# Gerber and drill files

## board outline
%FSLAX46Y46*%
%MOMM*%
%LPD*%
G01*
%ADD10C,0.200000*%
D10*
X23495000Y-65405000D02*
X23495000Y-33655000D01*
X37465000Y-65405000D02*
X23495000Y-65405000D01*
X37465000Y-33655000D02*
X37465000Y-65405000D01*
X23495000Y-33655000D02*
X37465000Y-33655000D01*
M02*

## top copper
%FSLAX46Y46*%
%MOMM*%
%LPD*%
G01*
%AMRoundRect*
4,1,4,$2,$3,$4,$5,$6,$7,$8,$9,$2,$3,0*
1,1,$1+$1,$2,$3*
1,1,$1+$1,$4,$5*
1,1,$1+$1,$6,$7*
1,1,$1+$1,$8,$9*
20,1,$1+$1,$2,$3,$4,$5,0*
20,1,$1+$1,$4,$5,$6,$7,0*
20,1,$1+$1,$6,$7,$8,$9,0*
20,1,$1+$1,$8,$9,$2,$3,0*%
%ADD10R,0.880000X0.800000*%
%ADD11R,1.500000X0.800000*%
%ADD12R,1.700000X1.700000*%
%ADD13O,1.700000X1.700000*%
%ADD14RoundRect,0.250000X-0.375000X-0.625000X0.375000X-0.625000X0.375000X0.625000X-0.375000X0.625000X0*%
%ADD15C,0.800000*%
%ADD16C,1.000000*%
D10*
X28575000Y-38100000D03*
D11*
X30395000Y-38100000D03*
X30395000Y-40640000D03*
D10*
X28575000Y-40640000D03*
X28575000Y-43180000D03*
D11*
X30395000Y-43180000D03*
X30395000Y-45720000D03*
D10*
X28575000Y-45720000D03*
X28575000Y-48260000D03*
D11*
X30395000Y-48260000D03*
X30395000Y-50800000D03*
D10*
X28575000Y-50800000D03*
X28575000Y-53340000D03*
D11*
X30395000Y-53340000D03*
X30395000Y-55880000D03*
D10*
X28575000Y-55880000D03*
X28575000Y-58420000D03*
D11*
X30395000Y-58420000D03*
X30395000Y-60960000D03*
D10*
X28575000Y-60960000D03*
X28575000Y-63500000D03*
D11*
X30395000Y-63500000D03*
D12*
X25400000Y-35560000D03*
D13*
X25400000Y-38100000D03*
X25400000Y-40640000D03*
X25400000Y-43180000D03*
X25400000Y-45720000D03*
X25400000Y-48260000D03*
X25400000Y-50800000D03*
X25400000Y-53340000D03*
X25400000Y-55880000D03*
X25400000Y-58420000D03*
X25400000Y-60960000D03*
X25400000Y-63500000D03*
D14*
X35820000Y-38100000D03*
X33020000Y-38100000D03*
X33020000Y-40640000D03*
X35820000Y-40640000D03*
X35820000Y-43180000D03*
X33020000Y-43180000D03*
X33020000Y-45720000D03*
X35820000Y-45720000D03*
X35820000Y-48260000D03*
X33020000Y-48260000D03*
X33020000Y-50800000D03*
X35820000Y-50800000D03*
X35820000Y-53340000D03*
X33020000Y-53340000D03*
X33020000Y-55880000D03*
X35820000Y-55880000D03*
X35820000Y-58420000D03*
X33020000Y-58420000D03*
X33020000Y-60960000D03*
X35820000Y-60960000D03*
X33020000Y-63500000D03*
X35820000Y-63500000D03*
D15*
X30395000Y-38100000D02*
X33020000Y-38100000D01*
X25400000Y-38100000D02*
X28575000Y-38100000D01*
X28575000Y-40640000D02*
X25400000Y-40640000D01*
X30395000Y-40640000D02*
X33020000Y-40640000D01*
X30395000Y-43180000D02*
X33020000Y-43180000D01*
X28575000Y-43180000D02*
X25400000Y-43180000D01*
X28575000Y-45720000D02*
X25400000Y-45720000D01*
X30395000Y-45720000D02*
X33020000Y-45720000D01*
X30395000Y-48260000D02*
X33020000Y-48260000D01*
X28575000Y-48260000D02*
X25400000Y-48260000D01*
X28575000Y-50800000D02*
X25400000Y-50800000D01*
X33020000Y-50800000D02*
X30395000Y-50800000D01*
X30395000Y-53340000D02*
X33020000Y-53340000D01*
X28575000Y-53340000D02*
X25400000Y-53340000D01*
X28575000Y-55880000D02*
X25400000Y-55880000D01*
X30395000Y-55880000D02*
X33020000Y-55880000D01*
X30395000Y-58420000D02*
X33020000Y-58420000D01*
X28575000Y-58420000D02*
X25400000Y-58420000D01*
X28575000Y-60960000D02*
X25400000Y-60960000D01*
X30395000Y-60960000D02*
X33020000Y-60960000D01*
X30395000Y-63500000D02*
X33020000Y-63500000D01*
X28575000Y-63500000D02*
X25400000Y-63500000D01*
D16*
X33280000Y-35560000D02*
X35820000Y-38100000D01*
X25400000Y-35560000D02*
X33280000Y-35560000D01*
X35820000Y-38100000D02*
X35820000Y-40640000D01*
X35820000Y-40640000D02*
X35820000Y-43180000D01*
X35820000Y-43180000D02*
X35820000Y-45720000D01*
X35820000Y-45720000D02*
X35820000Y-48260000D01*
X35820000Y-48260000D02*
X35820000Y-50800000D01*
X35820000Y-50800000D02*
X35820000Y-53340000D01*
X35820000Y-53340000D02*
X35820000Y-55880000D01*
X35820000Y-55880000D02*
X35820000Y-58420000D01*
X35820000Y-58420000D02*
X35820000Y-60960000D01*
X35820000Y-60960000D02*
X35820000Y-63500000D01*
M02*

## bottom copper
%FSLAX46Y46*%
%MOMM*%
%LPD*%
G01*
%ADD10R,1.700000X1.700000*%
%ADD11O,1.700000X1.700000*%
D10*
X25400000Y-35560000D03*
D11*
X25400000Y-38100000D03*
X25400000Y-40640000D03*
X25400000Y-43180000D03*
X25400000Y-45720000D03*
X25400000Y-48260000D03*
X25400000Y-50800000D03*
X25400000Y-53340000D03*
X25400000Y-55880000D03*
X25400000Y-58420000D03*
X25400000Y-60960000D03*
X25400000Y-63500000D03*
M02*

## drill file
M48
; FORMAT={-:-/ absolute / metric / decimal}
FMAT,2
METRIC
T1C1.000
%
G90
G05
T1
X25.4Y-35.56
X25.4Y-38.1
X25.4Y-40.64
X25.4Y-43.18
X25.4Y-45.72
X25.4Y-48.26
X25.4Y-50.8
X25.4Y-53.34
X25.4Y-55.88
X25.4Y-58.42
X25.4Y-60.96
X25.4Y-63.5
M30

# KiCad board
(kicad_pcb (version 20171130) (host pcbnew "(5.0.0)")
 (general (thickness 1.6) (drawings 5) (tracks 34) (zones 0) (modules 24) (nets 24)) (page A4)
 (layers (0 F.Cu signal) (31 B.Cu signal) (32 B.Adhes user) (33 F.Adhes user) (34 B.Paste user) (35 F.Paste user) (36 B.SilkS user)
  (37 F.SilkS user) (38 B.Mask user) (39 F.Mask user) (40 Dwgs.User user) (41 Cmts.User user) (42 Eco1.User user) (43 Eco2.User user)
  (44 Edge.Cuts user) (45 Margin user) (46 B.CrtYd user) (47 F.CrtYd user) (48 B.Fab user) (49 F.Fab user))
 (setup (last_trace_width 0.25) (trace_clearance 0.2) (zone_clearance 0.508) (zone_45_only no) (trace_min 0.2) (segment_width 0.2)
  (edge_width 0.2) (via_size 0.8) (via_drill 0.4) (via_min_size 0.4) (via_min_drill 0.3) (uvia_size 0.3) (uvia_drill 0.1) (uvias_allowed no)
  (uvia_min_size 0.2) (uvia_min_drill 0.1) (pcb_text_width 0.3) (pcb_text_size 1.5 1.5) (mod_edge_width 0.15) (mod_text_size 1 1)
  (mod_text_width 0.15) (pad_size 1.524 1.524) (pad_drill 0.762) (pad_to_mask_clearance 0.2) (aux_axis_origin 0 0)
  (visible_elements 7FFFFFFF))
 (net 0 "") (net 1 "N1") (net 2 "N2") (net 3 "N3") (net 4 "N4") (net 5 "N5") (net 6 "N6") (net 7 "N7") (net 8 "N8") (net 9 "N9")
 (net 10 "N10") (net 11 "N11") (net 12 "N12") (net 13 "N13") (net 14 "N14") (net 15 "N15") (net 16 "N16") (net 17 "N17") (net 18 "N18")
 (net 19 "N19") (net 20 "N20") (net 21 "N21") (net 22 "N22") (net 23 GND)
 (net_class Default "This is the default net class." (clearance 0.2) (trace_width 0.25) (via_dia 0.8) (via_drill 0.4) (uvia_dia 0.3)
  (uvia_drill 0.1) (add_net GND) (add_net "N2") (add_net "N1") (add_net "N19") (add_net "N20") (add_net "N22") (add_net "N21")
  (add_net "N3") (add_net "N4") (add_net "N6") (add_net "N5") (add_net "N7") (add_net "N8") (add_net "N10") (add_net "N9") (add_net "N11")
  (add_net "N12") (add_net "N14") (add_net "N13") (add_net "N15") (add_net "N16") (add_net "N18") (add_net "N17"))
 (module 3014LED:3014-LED (layer F.Cu) (at 28.575 38.1)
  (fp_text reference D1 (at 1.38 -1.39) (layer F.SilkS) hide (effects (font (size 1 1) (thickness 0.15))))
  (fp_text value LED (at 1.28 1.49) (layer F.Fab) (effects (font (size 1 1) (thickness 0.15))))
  (pad 2 smd rect (at 0 0) (size 0.88 0.8) (layers F.Cu F.Paste F.Mask) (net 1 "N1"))
  (pad 1 smd rect (at 1.82 0) (size 1.5 0.8) (layers F.Cu F.Paste F.Mask) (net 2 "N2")))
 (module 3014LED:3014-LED (layer F.Cu) (at 28.575 40.64)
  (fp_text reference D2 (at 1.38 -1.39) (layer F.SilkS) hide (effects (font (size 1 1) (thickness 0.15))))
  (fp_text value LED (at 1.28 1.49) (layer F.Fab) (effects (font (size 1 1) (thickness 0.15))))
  (pad 1 smd rect (at 1.82 0) (size 1.5 0.8) (layers F.Cu F.Paste F.Mask) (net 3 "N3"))
  (pad 2 smd rect (at 0 0) (size 0.88 0.8) (layers F.Cu F.Paste F.Mask) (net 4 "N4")))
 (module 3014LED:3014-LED (layer F.Cu) (at 28.575 43.18)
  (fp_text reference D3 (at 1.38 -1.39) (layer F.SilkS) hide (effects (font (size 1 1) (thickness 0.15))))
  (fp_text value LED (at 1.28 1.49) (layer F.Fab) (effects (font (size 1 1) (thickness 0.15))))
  (pad 2 smd rect (at 0 0) (size 0.88 0.8) (layers F.Cu F.Paste F.Mask) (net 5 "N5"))
  (pad 1 smd rect (at 1.82 0) (size 1.5 0.8) (layers F.Cu F.Paste F.Mask) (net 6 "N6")))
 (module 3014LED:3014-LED (layer F.Cu) (at 28.575 45.72)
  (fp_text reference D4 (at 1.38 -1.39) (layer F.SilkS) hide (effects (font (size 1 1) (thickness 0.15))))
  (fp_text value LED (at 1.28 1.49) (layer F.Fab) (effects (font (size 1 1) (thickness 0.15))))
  (pad 1 smd rect (at 1.82 0) (size 1.5 0.8) (layers F.Cu F.Paste F.Mask) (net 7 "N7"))
  (pad 2 smd rect (at 0 0) (size 0.88 0.8) (layers F.Cu F.Paste F.Mask) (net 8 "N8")))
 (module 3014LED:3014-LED (layer F.Cu) (at 28.575 48.26)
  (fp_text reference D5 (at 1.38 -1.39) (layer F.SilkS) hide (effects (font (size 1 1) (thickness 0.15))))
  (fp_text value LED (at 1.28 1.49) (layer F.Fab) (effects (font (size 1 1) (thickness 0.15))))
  (pad 2 smd rect (at 0 0) (size 0.88 0.8) (layers F.Cu F.Paste F.Mask) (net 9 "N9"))
  (pad 1 smd rect (at 1.82 0) (size 1.5 0.8) (layers F.Cu F.Paste F.Mask) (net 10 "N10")))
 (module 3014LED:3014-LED (layer F.Cu) (at 28.575 50.8)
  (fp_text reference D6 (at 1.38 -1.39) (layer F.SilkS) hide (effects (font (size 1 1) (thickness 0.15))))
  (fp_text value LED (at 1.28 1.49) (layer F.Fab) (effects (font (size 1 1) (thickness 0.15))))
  (pad 1 smd rect (at 1.82 0) (size 1.5 0.8) (layers F.Cu F.Paste F.Mask) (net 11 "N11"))
  (pad 2 smd rect (at 0 0) (size 0.88 0.8) (layers F.Cu F.Paste F.Mask) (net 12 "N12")))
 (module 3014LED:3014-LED (layer F.Cu) (at 28.575 53.34)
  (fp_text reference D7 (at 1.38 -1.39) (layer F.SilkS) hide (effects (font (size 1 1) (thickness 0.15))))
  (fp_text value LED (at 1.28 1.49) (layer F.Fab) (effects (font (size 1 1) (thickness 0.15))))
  (pad 2 smd rect (at 0 0) (size 0.88 0.8) (layers F.Cu F.Paste F.Mask) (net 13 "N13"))
  (pad 1 smd rect (at 1.82 0) (size 1.5 0.8) (layers F.Cu F.Paste F.Mask) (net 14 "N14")))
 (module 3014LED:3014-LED (layer F.Cu) (at 28.575 55.88)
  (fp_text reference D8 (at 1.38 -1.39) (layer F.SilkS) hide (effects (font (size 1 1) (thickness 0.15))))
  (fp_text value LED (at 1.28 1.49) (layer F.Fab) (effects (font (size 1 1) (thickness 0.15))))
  (pad 1 smd rect (at 1.82 0) (size 1.5 0.8) (layers F.Cu F.Paste F.Mask) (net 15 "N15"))
  (pad 2 smd rect (at 0 0) (size 0.88 0.8) (layers F.Cu F.Paste F.Mask) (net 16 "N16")))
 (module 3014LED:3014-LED (layer F.Cu) (at 28.575 58.42)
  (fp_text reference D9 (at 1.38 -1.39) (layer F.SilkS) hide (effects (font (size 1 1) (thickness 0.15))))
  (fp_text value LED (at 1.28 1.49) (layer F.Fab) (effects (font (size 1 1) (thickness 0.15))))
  (pad 2 smd rect (at 0 0) (size 0.88 0.8) (layers F.Cu F.Paste F.Mask) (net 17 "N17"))
  (pad 1 smd rect (at 1.82 0) (size 1.5 0.8) (layers F.Cu F.Paste F.Mask) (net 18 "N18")))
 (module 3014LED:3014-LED (layer F.Cu) (at 28.575 60.96)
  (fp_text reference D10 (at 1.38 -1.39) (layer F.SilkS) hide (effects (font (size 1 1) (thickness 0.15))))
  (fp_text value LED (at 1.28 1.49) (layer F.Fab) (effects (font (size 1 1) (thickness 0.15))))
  (pad 1 smd rect (at 1.82 0) (size 1.5 0.8) (layers F.Cu F.Paste F.Mask) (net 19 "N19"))
  (pad 2 smd rect (at 0 0) (size 0.88 0.8) (layers F.Cu F.Paste F.Mask) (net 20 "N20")))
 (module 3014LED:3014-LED (layer F.Cu) (at 28.575 63.5)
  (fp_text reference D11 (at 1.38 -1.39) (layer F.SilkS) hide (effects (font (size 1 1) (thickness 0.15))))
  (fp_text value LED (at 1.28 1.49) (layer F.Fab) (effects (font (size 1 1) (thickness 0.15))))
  (pad 2 smd rect (at 0 0) (size 0.88 0.8) (layers F.Cu F.Paste F.Mask) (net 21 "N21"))
  (pad 1 smd rect (at 1.82 0) (size 1.5 0.8) (layers F.Cu F.Paste F.Mask) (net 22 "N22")))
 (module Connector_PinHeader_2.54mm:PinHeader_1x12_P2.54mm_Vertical (layer F.Cu) (at 25.4 35.56)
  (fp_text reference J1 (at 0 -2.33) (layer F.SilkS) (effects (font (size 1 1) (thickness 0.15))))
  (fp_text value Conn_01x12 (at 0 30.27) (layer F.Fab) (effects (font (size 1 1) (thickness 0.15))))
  (pad 1 thru_hole rect (at 0 0) (size 1.7 1.7) (drill 1) (layers *.Cu *.Mask) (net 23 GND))
  (pad 2 thru_hole oval (at 0 2.54) (size 1.7 1.7) (drill 1) (layers *.Cu *.Mask) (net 1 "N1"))
  (pad 3 thru_hole oval (at 0 5.08) (size 1.7 1.7) (drill 1) (layers *.Cu *.Mask) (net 4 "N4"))
  (pad 4 thru_hole oval (at 0 7.62) (size 1.7 1.7) (drill 1) (layers *.Cu *.Mask) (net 5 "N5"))
  (pad 5 thru_hole oval (at 0 10.16) (size 1.7 1.7) (drill 1) (layers *.Cu *.Mask) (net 8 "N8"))
  (pad 6 thru_hole oval (at 0 12.7) (size 1.7 1.7) (drill 1) (layers *.Cu *.Mask) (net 9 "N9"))
  (pad 7 thru_hole oval (at 0 15.24) (size 1.7 1.7) (drill 1) (layers *.Cu *.Mask) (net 12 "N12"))
  (pad 8 thru_hole oval (at 0 17.78) (size 1.7 1.7) (drill 1) (layers *.Cu *.Mask) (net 13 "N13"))
  (pad 9 thru_hole oval (at 0 20.32) (size 1.7 1.7) (drill 1) (layers *.Cu *.Mask) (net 16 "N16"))
  (pad 10 thru_hole oval (at 0 22.86) (size 1.7 1.7) (drill 1) (layers *.Cu *.Mask) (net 17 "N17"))
  (pad 11 thru_hole oval (at 0 25.4) (size 1.7 1.7) (drill 1) (layers *.Cu *.Mask) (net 20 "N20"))
  (pad 12 thru_hole oval (at 0 27.94) (size 1.7 1.7) (drill 1) (layers *.Cu *.Mask) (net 21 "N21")))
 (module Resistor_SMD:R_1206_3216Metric (layer F.Cu) (at 34.42 38.1)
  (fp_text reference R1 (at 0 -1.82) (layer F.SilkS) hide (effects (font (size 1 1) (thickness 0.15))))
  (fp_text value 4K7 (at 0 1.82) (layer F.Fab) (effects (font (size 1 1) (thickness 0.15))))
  (pad 2 smd roundrect (at 1.4 0) (size 1.25 1.75) (layers F.Cu F.Paste F.Mask) (roundrect_rratio 0.2) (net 23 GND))
  (pad 1 smd roundrect (at -1.4 0) (size 1.25 1.75) (layers F.Cu F.Paste F.Mask) (roundrect_rratio 0.2) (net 2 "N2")))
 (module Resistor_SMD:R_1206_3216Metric (layer F.Cu) (at 34.42 40.64)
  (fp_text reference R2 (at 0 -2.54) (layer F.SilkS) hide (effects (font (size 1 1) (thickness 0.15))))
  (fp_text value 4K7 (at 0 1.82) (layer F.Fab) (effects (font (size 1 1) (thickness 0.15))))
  (pad 1 smd roundrect (at -1.4 0) (size 1.25 1.75) (layers F.Cu F.Paste F.Mask) (roundrect_rratio 0.2) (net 3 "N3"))
  (pad 2 smd roundrect (at 1.4 0) (size 1.25 1.75) (layers F.Cu F.Paste F.Mask) (roundrect_rratio 0.2) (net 23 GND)))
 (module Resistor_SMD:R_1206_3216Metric (layer F.Cu) (at 34.42 43.18)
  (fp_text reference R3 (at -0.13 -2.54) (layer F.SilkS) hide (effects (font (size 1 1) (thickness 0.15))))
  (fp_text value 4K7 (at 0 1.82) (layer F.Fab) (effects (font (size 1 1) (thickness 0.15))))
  (pad 2 smd roundrect (at 1.4 0) (size 1.25 1.75) (layers F.Cu F.Paste F.Mask) (roundrect_rratio 0.2) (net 23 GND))
  (pad 1 smd roundrect (at -1.4 0) (size 1.25 1.75) (layers F.Cu F.Paste F.Mask) (roundrect_rratio 0.2) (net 6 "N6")))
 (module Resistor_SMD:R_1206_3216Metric (layer F.Cu) (at 34.42 45.72)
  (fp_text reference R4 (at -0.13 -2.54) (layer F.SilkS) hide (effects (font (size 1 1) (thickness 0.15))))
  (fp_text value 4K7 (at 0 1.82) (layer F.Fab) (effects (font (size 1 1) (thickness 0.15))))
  (pad 1 smd roundrect (at -1.4 0) (size 1.25 1.75) (layers F.Cu F.Paste F.Mask) (roundrect_rratio 0.2) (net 7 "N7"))
  (pad 2 smd roundrect (at 1.4 0) (size 1.25 1.75) (layers F.Cu F.Paste F.Mask) (roundrect_rratio 0.2) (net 23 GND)))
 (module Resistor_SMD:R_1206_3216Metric (layer F.Cu) (at 34.42 48.26)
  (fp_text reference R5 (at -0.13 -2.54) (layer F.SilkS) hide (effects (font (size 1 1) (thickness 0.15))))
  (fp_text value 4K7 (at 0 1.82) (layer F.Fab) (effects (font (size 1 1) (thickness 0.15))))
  (pad 2 smd roundrect (at 1.4 0) (size 1.25 1.75) (layers F.Cu F.Paste F.Mask) (roundrect_rratio 0.2) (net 23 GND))
  (pad 1 smd roundrect (at -1.4 0) (size 1.25 1.75) (layers F.Cu F.Paste F.Mask) (roundrect_rratio 0.2) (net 10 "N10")))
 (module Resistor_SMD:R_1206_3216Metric (layer F.Cu) (at 34.42 50.8)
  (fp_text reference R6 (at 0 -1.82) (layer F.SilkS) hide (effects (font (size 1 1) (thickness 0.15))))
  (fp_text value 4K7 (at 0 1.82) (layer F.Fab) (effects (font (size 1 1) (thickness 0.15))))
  (pad 1 smd roundrect (at -1.4 0) (size 1.25 1.75) (layers F.Cu F.Paste F.Mask) (roundrect_rratio 0.2) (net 11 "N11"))
  (pad 2 smd roundrect (at 1.4 0) (size 1.25 1.75) (layers F.Cu F.Paste F.Mask) (roundrect_rratio 0.2) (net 23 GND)))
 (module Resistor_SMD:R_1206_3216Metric (layer F.Cu) (at 34.42 53.34)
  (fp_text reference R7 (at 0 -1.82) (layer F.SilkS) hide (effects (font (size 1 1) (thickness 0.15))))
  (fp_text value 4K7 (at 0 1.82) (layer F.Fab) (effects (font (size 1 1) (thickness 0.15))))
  (pad 2 smd roundrect (at 1.4 0) (size 1.25 1.75) (layers F.Cu F.Paste F.Mask) (roundrect_rratio 0.2) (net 23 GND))
  (pad 1 smd roundrect (at -1.4 0) (size 1.25 1.75) (layers F.Cu F.Paste F.Mask) (roundrect_rratio 0.2) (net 14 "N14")))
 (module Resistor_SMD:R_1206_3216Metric (layer F.Cu) (at 34.42 55.88)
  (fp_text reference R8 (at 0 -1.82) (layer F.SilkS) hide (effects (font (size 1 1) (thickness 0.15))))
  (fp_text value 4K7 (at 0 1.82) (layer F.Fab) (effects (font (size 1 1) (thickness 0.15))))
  (pad 1 smd roundrect (at -1.4 0) (size 1.25 1.75) (layers F.Cu F.Paste F.Mask) (roundrect_rratio 0.2) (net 15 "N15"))
  (pad 2 smd roundrect (at 1.4 0) (size 1.25 1.75) (layers F.Cu F.Paste F.Mask) (roundrect_rratio 0.2) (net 23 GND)))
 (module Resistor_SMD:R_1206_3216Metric (layer F.Cu) (at 34.42 58.42)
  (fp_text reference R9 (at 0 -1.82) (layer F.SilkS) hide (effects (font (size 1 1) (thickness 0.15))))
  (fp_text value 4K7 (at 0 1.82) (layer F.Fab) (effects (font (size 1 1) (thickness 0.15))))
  (pad 2 smd roundrect (at 1.4 0) (size 1.25 1.75) (layers F.Cu F.Paste F.Mask) (roundrect_rratio 0.2) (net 23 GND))
  (pad 1 smd roundrect (at -1.4 0) (size 1.25 1.75) (layers F.Cu F.Paste F.Mask) (roundrect_rratio 0.2) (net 18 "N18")))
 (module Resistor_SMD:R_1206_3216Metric (layer F.Cu) (at 34.42 60.96)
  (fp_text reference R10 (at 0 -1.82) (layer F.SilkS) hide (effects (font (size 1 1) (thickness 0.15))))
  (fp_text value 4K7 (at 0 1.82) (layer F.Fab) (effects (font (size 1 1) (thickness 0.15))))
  (pad 1 smd roundrect (at -1.4 0) (size 1.25 1.75) (layers F.Cu F.Paste F.Mask) (roundrect_rratio 0.2) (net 19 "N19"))
  (pad 2 smd roundrect (at 1.4 0) (size 1.25 1.75) (layers F.Cu F.Paste F.Mask) (roundrect_rratio 0.2) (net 23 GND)))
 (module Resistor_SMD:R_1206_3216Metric (layer F.Cu) (at 34.42 63.5)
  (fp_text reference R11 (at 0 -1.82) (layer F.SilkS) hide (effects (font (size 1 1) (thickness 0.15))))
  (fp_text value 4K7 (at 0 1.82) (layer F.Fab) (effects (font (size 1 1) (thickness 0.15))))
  (pad 1 smd roundrect (at -1.4 0) (size 1.25 1.75) (layers F.Cu F.Paste F.Mask) (roundrect_rratio 0.2) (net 22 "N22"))
  (pad 2 smd roundrect (at 1.4 0) (size 1.25 1.75) (layers F.Cu F.Paste F.Mask) (roundrect_rratio 0.2) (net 23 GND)))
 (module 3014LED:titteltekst (layer B.Cu) (at 31.75 49.53 90)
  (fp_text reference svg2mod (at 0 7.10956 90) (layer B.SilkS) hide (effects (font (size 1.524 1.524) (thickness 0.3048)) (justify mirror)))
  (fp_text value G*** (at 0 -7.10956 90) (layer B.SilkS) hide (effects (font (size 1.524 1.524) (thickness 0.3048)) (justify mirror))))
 (gr_line (start 23.495 65.405) (end 23.495 33.655) (layer Edge.Cuts) (width 0.2))
 (gr_line (start 37.465 65.405) (end 23.495 65.405) (layer Edge.Cuts) (width 0.2))
 (gr_line (start 37.465 33.655) (end 37.465 65.405) (layer Edge.Cuts) (width 0.2))
 (gr_line (start 23.495 33.655) (end 37.465 33.655) (layer Edge.Cuts) (width 0.2))
 (segment (start 30.395 38.1) (end 33.02 38.1) (width 0.8) (layer F.Cu) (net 2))
 (segment (start 25.4 38.1) (end 28.575 38.1) (width 0.8) (layer F.Cu) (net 1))
 (segment (start 28.575 40.64) (end 25.4 40.64) (width 0.8) (layer F.Cu) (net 4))
 (segment (start 30.395 40.64) (end 33.02 40.64) (width 0.8) (layer F.Cu) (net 3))
 (segment (start 30.395 43.18) (end 33.02 43.18) (width 0.8) (layer F.Cu) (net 6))
 (segment (start 28.575 43.18) (end 25.4 43.18) (width 0.8) (layer F.Cu) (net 5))
 (segment (start 28.575 45.72) (end 25.4 45.72) (width 0.8) (layer F.Cu) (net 8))
 (segment (start 30.395 45.72) (end 33.02 45.72) (width 0.8) (layer F.Cu) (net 7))
 (segment (start 30.395 48.26) (end 33.02 48.26) (width 0.8) (layer F.Cu) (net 10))
 (segment (start 28.575 48.26) (end 25.4 48.26) (width 0.8) (layer F.Cu) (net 9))
 (segment (start 28.575 50.8) (end 25.4 50.8) (width 0.8) (layer F.Cu) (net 12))
 (segment (start 33.02 50.8) (end 30.395 50.8) (width 0.8) (layer F.Cu) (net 11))
 (segment (start 30.395 53.34) (end 33.02 53.34) (width 0.8) (layer F.Cu) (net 14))
 (segment (start 28.575 53.34) (end 25.4 53.34) (width 0.8) (layer F.Cu) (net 13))
 (segment (start 28.575 55.88) (end 25.4 55.88) (width 0.8) (layer F.Cu) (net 16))
 (segment (start 30.395 55.88) (end 33.02 55.88) (width 0.8) (layer F.Cu) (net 15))
 (segment (start 30.395 58.42) (end 33.02 58.42) (width 0.8) (layer F.Cu) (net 18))
 (segment (start 28.575 58.42) (end 25.4 58.42) (width 0.8) (layer F.Cu) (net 17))
 (segment (start 28.575 60.96) (end 25.4 60.96) (width 0.8) (layer F.Cu) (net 20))
 (segment (start 30.395 60.96) (end 33.02 60.96) (width 0.8) (layer F.Cu) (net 19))
 (segment (start 30.395 63.5) (end 33.02 63.5) (width 0.8) (layer F.Cu) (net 22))
 (segment (start 28.575 63.5) (end 25.4 63.5) (width 0.8) (layer F.Cu) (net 21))
 (segment (start 33.28 35.56) (end 35.82 38.1) (width 1) (layer F.Cu) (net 23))
 (segment (start 25.4 35.56) (end 33.28 35.56) (width 1) (layer F.Cu) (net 23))
 (segment (start 35.82 38.1) (end 35.82 40.64) (width 1) (layer F.Cu) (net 23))
 (segment (start 35.82 40.64) (end 35.82 43.18) (width 1) (layer F.Cu) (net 23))
 (segment (start 35.82 43.18) (end 35.82 45.72) (width 1) (layer F.Cu) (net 23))
 (segment (start 35.82 45.72) (end 35.82 48.26) (width 1) (layer F.Cu) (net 23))
 (segment (start 35.82 48.26) (end 35.82 50.8) (width 1) (layer F.Cu) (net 23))
 (segment (start 35.82 50.8) (end 35.82 53.34) (width 1) (layer F.Cu) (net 23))
 (segment (start 35.82 53.34) (end 35.82 55.88) (width 1) (layer F.Cu) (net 23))
 (segment (start 35.82 55.88) (end 35.82 58.42) (width 1) (layer F.Cu) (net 23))
 (segment (start 35.82 58.42) (end 35.82 60.96) (width 1) (layer F.Cu) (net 23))
 (segment (start 35.82 60.96) (end 35.82 63.5) (width 1) (layer F.Cu) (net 23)))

